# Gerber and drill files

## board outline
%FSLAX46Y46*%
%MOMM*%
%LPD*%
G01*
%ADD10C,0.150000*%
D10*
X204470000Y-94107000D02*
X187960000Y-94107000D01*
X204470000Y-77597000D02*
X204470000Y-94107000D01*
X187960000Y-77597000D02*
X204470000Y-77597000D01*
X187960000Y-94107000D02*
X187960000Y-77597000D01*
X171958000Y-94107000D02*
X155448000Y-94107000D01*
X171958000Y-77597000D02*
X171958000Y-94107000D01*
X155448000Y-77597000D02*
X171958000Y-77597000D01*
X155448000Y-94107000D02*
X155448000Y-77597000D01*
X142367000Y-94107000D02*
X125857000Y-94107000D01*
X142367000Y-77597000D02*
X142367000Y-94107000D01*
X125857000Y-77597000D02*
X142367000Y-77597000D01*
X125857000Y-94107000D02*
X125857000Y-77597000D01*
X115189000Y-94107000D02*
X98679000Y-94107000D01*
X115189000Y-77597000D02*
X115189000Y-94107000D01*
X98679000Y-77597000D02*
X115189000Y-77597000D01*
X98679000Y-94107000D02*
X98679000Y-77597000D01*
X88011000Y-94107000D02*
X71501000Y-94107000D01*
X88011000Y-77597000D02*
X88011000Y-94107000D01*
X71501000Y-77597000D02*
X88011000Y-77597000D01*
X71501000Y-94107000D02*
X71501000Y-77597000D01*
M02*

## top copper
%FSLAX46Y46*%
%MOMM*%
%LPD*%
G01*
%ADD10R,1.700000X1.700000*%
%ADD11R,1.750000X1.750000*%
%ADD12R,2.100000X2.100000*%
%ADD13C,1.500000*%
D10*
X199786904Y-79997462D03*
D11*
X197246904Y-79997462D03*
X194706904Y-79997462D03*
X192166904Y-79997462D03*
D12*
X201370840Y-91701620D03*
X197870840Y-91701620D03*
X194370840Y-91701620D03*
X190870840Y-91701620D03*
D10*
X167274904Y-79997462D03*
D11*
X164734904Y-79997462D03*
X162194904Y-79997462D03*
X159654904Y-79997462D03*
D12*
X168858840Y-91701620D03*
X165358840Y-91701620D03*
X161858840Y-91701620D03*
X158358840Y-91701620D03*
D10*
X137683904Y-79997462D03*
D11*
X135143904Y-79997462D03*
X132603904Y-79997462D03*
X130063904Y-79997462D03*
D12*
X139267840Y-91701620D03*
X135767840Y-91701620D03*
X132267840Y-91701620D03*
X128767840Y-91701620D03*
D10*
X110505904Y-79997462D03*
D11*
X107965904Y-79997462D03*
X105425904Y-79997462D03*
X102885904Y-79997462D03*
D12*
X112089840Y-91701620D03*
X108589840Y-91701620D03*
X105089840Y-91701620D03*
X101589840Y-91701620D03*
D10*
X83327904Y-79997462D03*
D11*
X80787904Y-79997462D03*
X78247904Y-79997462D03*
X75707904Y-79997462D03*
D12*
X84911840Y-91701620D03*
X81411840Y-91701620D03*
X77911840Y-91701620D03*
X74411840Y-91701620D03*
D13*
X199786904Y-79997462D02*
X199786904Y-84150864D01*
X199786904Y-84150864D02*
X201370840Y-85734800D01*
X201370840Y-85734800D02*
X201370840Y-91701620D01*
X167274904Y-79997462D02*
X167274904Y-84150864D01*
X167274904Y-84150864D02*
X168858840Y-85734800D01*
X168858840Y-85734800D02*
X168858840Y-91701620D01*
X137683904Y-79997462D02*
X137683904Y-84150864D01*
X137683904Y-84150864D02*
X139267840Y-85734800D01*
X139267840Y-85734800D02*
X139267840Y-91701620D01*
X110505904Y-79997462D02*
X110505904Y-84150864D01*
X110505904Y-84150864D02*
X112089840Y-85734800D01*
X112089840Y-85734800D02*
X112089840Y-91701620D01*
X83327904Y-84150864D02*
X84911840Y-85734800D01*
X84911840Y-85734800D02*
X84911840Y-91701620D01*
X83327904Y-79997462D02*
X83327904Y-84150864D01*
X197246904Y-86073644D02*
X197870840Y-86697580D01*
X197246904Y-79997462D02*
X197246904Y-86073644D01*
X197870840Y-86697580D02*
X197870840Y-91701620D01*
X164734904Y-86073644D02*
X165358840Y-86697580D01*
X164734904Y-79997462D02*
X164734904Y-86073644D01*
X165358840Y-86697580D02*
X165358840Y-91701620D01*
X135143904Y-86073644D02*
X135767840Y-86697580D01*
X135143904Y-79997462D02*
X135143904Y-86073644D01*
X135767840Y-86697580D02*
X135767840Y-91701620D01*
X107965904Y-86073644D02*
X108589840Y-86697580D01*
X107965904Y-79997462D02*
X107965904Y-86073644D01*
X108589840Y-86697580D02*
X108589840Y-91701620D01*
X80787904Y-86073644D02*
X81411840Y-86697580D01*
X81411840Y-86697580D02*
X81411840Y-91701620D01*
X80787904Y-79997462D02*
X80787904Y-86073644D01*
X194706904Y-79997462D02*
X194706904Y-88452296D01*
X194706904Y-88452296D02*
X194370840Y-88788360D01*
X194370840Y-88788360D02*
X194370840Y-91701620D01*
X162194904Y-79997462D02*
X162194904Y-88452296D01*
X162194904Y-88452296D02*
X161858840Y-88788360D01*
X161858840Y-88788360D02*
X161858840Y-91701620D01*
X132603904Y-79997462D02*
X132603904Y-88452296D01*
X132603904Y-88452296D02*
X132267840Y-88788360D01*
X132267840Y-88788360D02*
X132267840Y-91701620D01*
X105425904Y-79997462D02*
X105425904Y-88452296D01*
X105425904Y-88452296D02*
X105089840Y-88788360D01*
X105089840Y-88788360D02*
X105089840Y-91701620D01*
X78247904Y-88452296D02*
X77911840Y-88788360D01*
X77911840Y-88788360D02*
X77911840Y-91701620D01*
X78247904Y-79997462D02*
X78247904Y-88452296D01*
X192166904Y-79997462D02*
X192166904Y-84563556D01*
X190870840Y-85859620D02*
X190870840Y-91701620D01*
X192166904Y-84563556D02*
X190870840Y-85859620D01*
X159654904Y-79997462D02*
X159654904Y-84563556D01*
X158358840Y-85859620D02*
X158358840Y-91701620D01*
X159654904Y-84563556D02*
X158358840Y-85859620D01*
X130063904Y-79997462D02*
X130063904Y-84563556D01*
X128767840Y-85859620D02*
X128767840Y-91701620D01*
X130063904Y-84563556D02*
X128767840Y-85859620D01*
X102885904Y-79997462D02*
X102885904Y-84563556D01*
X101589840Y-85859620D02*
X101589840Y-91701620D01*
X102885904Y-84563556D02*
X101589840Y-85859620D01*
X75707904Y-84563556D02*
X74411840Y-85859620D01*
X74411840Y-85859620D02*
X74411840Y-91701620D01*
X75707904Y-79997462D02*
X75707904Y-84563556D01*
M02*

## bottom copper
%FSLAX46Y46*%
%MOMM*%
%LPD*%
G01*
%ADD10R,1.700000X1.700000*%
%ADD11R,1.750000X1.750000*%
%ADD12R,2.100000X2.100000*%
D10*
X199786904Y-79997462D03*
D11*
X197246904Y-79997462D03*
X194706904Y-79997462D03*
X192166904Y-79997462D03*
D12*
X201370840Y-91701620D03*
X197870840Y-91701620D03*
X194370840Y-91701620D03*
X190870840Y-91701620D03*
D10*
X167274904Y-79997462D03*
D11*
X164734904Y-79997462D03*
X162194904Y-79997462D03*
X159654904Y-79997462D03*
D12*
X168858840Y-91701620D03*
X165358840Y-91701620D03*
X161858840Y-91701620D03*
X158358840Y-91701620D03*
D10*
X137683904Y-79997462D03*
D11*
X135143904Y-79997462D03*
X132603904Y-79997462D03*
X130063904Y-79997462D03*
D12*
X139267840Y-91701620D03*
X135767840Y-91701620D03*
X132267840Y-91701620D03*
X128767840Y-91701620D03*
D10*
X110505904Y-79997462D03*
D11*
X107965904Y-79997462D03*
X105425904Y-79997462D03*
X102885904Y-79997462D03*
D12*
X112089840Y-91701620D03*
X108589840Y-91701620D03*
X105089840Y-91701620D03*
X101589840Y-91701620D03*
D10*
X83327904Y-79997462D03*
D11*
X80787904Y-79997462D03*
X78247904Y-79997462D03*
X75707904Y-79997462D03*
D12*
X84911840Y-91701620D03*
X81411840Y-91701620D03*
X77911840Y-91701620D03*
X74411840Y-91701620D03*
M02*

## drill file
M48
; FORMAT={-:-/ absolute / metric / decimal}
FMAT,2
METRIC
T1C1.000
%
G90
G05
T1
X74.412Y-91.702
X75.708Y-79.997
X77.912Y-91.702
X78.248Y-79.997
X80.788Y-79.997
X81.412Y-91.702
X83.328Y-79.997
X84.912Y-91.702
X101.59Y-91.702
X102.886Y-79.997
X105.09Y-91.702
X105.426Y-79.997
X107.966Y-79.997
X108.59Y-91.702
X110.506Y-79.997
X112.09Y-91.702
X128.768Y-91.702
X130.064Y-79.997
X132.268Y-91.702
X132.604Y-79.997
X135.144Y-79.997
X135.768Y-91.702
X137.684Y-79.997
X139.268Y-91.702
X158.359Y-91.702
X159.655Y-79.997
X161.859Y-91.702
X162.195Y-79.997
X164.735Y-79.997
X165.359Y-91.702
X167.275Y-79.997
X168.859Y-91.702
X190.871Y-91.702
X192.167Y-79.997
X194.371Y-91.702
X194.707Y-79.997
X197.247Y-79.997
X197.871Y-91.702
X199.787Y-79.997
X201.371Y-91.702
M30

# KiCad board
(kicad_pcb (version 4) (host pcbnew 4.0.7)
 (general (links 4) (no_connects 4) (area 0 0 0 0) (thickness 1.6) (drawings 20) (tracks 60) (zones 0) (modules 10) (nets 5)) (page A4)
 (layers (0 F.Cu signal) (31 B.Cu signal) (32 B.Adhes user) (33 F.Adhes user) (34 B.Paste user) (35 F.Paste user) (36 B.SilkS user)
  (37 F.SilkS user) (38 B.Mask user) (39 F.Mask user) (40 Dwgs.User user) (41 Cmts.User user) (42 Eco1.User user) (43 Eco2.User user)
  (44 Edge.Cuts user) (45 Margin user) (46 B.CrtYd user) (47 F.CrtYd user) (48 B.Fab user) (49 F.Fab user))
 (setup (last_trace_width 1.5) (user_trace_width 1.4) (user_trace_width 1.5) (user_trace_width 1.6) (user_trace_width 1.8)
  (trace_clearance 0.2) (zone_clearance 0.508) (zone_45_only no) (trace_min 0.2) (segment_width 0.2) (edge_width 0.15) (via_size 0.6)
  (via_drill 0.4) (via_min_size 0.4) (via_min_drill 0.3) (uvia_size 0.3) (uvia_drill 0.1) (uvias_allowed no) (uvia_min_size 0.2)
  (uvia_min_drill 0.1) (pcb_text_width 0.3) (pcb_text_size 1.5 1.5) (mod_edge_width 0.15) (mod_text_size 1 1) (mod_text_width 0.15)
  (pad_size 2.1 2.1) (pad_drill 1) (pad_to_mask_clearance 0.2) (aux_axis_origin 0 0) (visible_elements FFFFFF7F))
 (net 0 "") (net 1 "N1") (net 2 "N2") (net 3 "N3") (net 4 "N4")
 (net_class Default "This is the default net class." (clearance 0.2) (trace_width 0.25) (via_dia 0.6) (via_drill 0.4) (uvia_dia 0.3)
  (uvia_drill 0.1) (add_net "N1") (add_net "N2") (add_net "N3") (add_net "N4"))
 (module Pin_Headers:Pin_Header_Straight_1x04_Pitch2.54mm (layer F.Cu) (at 199.786904 79.997462 270)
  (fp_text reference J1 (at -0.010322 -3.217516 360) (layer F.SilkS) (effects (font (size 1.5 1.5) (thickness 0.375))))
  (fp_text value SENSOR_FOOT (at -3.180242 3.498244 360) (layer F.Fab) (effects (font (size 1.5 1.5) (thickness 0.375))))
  (pad 1 thru_hole rect (at 0 0 270) (size 1.7 1.7) (drill 1) (layers *.Cu *.Mask) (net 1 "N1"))
  (pad 2 thru_hole rect (at 0 2.54 270) (size 1.75 1.75) (drill 1) (layers *.Cu *.Mask) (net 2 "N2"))
  (pad 3 thru_hole rect (at 0 5.08 270) (size 1.75 1.75) (drill 1) (layers *.Cu *.Mask) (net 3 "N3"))
  (pad 4 thru_hole rect (at 0 7.62 270) (size 1.75 1.75) (drill 1) (layers *.Cu *.Mask) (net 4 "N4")))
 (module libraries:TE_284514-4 (layer F.Cu) (at 196.12084 91.70162 180)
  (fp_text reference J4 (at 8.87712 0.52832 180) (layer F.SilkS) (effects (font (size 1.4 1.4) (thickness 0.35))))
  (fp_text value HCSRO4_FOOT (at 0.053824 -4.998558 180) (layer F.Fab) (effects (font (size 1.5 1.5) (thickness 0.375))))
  (pad 1 thru_hole rect (at -5.25 0 180) (size 2.1 2.1) (drill 1) (layers *.Cu *.Mask) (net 1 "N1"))
  (pad 2 thru_hole rect (at -1.75 0 180) (size 2.1 2.1) (drill 1) (layers *.Cu *.Mask) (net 2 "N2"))
  (pad 3 thru_hole rect (at 1.75 0 180) (size 2.1 2.1) (drill 1) (layers *.Cu *.Mask) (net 3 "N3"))
  (pad 4 thru_hole rect (at 5.25 0 180) (size 2.1 2.1) (drill 1) (layers *.Cu *.Mask) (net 4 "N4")))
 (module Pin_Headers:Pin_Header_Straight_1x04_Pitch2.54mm (layer F.Cu) (at 167.274904 79.997462 270)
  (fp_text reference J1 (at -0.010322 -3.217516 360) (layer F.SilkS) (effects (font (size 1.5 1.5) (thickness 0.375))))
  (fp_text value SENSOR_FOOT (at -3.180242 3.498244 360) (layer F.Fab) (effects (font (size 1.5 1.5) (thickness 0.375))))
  (pad 1 thru_hole rect (at 0 0 270) (size 1.7 1.7) (drill 1) (layers *.Cu *.Mask) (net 1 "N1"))
  (pad 2 thru_hole rect (at 0 2.54 270) (size 1.75 1.75) (drill 1) (layers *.Cu *.Mask) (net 2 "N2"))
  (pad 3 thru_hole rect (at 0 5.08 270) (size 1.75 1.75) (drill 1) (layers *.Cu *.Mask) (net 3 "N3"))
  (pad 4 thru_hole rect (at 0 7.62 270) (size 1.75 1.75) (drill 1) (layers *.Cu *.Mask) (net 4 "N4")))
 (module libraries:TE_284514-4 (layer F.Cu) (at 163.60884 91.70162 180)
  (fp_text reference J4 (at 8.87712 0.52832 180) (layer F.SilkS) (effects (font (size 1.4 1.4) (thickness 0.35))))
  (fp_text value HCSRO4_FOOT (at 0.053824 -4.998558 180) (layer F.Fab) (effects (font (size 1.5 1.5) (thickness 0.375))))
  (pad 1 thru_hole rect (at -5.25 0 180) (size 2.1 2.1) (drill 1) (layers *.Cu *.Mask) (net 1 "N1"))
  (pad 2 thru_hole rect (at -1.75 0 180) (size 2.1 2.1) (drill 1) (layers *.Cu *.Mask) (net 2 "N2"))
  (pad 3 thru_hole rect (at 1.75 0 180) (size 2.1 2.1) (drill 1) (layers *.Cu *.Mask) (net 3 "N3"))
  (pad 4 thru_hole rect (at 5.25 0 180) (size 2.1 2.1) (drill 1) (layers *.Cu *.Mask) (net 4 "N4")))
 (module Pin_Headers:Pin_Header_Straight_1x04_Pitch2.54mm (layer F.Cu) (at 137.683904 79.997462 270)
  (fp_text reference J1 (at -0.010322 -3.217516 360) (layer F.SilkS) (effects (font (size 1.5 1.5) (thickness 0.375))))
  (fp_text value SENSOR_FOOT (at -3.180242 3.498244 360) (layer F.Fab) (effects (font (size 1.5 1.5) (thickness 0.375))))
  (pad 1 thru_hole rect (at 0 0 270) (size 1.7 1.7) (drill 1) (layers *.Cu *.Mask) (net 1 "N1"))
  (pad 2 thru_hole rect (at 0 2.54 270) (size 1.75 1.75) (drill 1) (layers *.Cu *.Mask) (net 2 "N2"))
  (pad 3 thru_hole rect (at 0 5.08 270) (size 1.75 1.75) (drill 1) (layers *.Cu *.Mask) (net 3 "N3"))
  (pad 4 thru_hole rect (at 0 7.62 270) (size 1.75 1.75) (drill 1) (layers *.Cu *.Mask) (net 4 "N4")))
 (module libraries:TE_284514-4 (layer F.Cu) (at 134.01784 91.70162 180)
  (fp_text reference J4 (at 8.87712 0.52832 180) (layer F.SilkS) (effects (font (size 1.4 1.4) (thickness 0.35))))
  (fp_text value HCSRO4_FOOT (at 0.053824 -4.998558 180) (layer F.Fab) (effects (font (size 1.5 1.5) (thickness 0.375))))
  (pad 1 thru_hole rect (at -5.25 0 180) (size 2.1 2.1) (drill 1) (layers *.Cu *.Mask) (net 1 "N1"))
  (pad 2 thru_hole rect (at -1.75 0 180) (size 2.1 2.1) (drill 1) (layers *.Cu *.Mask) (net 2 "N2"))
  (pad 3 thru_hole rect (at 1.75 0 180) (size 2.1 2.1) (drill 1) (layers *.Cu *.Mask) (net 3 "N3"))
  (pad 4 thru_hole rect (at 5.25 0 180) (size 2.1 2.1) (drill 1) (layers *.Cu *.Mask) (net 4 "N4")))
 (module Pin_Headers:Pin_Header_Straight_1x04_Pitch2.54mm (layer F.Cu) (at 110.505904 79.997462 270)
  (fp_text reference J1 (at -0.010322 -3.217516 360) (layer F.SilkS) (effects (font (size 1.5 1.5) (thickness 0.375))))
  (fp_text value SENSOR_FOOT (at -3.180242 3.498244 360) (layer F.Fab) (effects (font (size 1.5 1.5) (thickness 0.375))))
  (pad 1 thru_hole rect (at 0 0 270) (size 1.7 1.7) (drill 1) (layers *.Cu *.Mask) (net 1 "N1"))
  (pad 2 thru_hole rect (at 0 2.54 270) (size 1.75 1.75) (drill 1) (layers *.Cu *.Mask) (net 2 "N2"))
  (pad 3 thru_hole rect (at 0 5.08 270) (size 1.75 1.75) (drill 1) (layers *.Cu *.Mask) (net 3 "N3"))
  (pad 4 thru_hole rect (at 0 7.62 270) (size 1.75 1.75) (drill 1) (layers *.Cu *.Mask) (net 4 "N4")))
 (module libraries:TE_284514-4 (layer F.Cu) (at 106.83984 91.70162 180)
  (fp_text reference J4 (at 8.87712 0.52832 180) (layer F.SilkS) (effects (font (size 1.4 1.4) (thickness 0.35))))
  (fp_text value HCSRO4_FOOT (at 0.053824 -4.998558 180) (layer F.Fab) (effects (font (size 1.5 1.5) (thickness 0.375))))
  (pad 1 thru_hole rect (at -5.25 0 180) (size 2.1 2.1) (drill 1) (layers *.Cu *.Mask) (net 1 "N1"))
  (pad 2 thru_hole rect (at -1.75 0 180) (size 2.1 2.1) (drill 1) (layers *.Cu *.Mask) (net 2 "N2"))
  (pad 3 thru_hole rect (at 1.75 0 180) (size 2.1 2.1) (drill 1) (layers *.Cu *.Mask) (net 3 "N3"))
  (pad 4 thru_hole rect (at 5.25 0 180) (size 2.1 2.1) (drill 1) (layers *.Cu *.Mask) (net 4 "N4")))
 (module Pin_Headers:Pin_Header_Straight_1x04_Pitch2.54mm (layer F.Cu) (at 83.327904 79.997462 270)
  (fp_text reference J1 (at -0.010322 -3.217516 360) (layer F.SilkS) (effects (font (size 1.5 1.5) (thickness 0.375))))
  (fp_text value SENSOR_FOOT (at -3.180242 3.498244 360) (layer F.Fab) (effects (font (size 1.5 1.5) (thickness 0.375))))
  (pad 1 thru_hole rect (at 0 0 270) (size 1.7 1.7) (drill 1) (layers *.Cu *.Mask) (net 1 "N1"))
  (pad 2 thru_hole rect (at 0 2.54 270) (size 1.75 1.75) (drill 1) (layers *.Cu *.Mask) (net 2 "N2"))
  (pad 3 thru_hole rect (at 0 5.08 270) (size 1.75 1.75) (drill 1) (layers *.Cu *.Mask) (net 3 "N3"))
  (pad 4 thru_hole rect (at 0 7.62 270) (size 1.75 1.75) (drill 1) (layers *.Cu *.Mask) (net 4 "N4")))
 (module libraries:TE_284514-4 (layer F.Cu) (at 79.66184 91.70162 180)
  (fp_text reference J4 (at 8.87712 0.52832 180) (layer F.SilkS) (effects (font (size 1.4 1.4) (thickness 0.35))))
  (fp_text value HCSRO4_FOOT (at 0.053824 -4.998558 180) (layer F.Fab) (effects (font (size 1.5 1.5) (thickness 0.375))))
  (pad 1 thru_hole rect (at -5.25 0 180) (size 2.1 2.1) (drill 1) (layers *.Cu *.Mask) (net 1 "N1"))
  (pad 2 thru_hole rect (at -1.75 0 180) (size 2.1 2.1) (drill 1) (layers *.Cu *.Mask) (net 2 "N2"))
  (pad 3 thru_hole rect (at 1.75 0 180) (size 2.1 2.1) (drill 1) (layers *.Cu *.Mask) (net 3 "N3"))
  (pad 4 thru_hole rect (at 5.25 0 180) (size 2.1 2.1) (drill 1) (layers *.Cu *.Mask) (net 4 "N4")))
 (gr_line (start 204.47 94.107) (end 187.96 94.107) (layer Edge.Cuts) (width 0.15))
 (gr_line (start 204.47 77.597) (end 204.47 94.107) (layer Edge.Cuts) (width 0.15))
 (gr_line (start 187.96 77.597) (end 204.47 77.597) (layer Edge.Cuts) (width 0.15))
 (gr_line (start 187.96 94.107) (end 187.96 77.597) (layer Edge.Cuts) (width 0.15))
 (gr_line (start 171.958 94.107) (end 155.448 94.107) (layer Edge.Cuts) (width 0.15))
 (gr_line (start 171.958 77.597) (end 171.958 94.107) (layer Edge.Cuts) (width 0.15))
 (gr_line (start 155.448 77.597) (end 171.958 77.597) (layer Edge.Cuts) (width 0.15))
 (gr_line (start 155.448 94.107) (end 155.448 77.597) (layer Edge.Cuts) (width 0.15))
 (gr_line (start 142.367 94.107) (end 125.857 94.107) (layer Edge.Cuts) (width 0.15))
 (gr_line (start 142.367 77.597) (end 142.367 94.107) (layer Edge.Cuts) (width 0.15))
 (gr_line (start 125.857 77.597) (end 142.367 77.597) (layer Edge.Cuts) (width 0.15))
 (gr_line (start 125.857 94.107) (end 125.857 77.597) (layer Edge.Cuts) (width 0.15))
 (gr_line (start 115.189 94.107) (end 98.679 94.107) (layer Edge.Cuts) (width 0.15))
 (gr_line (start 115.189 77.597) (end 115.189 94.107) (layer Edge.Cuts) (width 0.15))
 (gr_line (start 98.679 77.597) (end 115.189 77.597) (layer Edge.Cuts) (width 0.15))
 (gr_line (start 98.679 94.107) (end 98.679 77.597) (layer Edge.Cuts) (width 0.15))
 (gr_line (start 88.011 94.107) (end 71.501 94.107) (layer Edge.Cuts) (width 0.15))
 (gr_line (start 88.011 77.597) (end 88.011 94.107) (layer Edge.Cuts) (width 0.15))
 (gr_line (start 71.501 77.597) (end 88.011 77.597) (layer Edge.Cuts) (width 0.15))
 (gr_line (start 71.501 94.107) (end 71.501 77.597) (layer Edge.Cuts) (width 0.15))
 (segment (start 199.786904 79.997462) (end 199.786904 84.150864) (width 1.5) (layer F.Cu) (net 1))
 (segment (start 199.786904 84.150864) (end 201.37084 85.7348) (width 1.5) (layer F.Cu) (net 1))
 (segment (start 201.37084 85.7348) (end 201.37084 91.70162) (width 1.5) (layer F.Cu) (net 1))
 (segment (start 167.274904 79.997462) (end 167.274904 84.150864) (width 1.5) (layer F.Cu) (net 1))
 (segment (start 167.274904 84.150864) (end 168.85884 85.7348) (width 1.5) (layer F.Cu) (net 1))
 (segment (start 168.85884 85.7348) (end 168.85884 91.70162) (width 1.5) (layer F.Cu) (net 1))
 (segment (start 137.683904 79.997462) (end 137.683904 84.150864) (width 1.5) (layer F.Cu) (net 1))
 (segment (start 137.683904 84.150864) (end 139.26784 85.7348) (width 1.5) (layer F.Cu) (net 1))
 (segment (start 139.26784 85.7348) (end 139.26784 91.70162) (width 1.5) (layer F.Cu) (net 1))
 (segment (start 110.505904 79.997462) (end 110.505904 84.150864) (width 1.5) (layer F.Cu) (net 1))
 (segment (start 110.505904 84.150864) (end 112.08984 85.7348) (width 1.5) (layer F.Cu) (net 1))
 (segment (start 112.08984 85.7348) (end 112.08984 91.70162) (width 1.5) (layer F.Cu) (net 1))
 (segment (start 83.327904 84.150864) (end 84.91184 85.7348) (width 1.5) (layer F.Cu) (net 1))
 (segment (start 84.91184 85.7348) (end 84.91184 91.70162) (width 1.5) (layer F.Cu) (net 1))
 (segment (start 83.327904 79.997462) (end 83.327904 84.150864) (width 1.5) (layer F.Cu) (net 1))
 (segment (start 197.246904 86.073644) (end 197.87084 86.69758) (width 1.5) (layer F.Cu) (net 2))
 (segment (start 197.246904 79.997462) (end 197.246904 86.073644) (width 1.5) (layer F.Cu) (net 2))
 (segment (start 197.87084 86.69758) (end 197.87084 91.70162) (width 1.5) (layer F.Cu) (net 2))
 (segment (start 164.734904 86.073644) (end 165.35884 86.69758) (width 1.5) (layer F.Cu) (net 2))
 (segment (start 164.734904 79.997462) (end 164.734904 86.073644) (width 1.5) (layer F.Cu) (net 2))
 (segment (start 165.35884 86.69758) (end 165.35884 91.70162) (width 1.5) (layer F.Cu) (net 2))
 (segment (start 135.143904 86.073644) (end 135.76784 86.69758) (width 1.5) (layer F.Cu) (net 2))
 (segment (start 135.143904 79.997462) (end 135.143904 86.073644) (width 1.5) (layer F.Cu) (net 2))
 (segment (start 135.76784 86.69758) (end 135.76784 91.70162) (width 1.5) (layer F.Cu) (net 2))
 (segment (start 107.965904 86.073644) (end 108.58984 86.69758) (width 1.5) (layer F.Cu) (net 2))
 (segment (start 107.965904 79.997462) (end 107.965904 86.073644) (width 1.5) (layer F.Cu) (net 2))
 (segment (start 108.58984 86.69758) (end 108.58984 91.70162) (width 1.5) (layer F.Cu) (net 2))
 (segment (start 80.787904 86.073644) (end 81.41184 86.69758) (width 1.5) (layer F.Cu) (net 2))
 (segment (start 81.41184 86.69758) (end 81.41184 91.70162) (width 1.5) (layer F.Cu) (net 2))
 (segment (start 80.787904 79.997462) (end 80.787904 86.073644) (width 1.5) (layer F.Cu) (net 2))
 (segment (start 194.706904 79.997462) (end 194.706904 88.452296) (width 1.5) (layer F.Cu) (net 3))
 (segment (start 194.706904 88.452296) (end 194.37084 88.78836) (width 1.5) (layer F.Cu) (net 3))
 (segment (start 194.37084 88.78836) (end 194.37084 91.70162) (width 1.5) (layer F.Cu) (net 3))
 (segment (start 162.194904 79.997462) (end 162.194904 88.452296) (width 1.5) (layer F.Cu) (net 3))
 (segment (start 162.194904 88.452296) (end 161.85884 88.78836) (width 1.5) (layer F.Cu) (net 3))
 (segment (start 161.85884 88.78836) (end 161.85884 91.70162) (width 1.5) (layer F.Cu) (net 3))
 (segment (start 132.603904 79.997462) (end 132.603904 88.452296) (width 1.5) (layer F.Cu) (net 3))
 (segment (start 132.603904 88.452296) (end 132.26784 88.78836) (width 1.5) (layer F.Cu) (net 3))
 (segment (start 132.26784 88.78836) (end 132.26784 91.70162) (width 1.5) (layer F.Cu) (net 3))
 (segment (start 105.425904 79.997462) (end 105.425904 88.452296) (width 1.5) (layer F.Cu) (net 3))
 (segment (start 105.425904 88.452296) (end 105.08984 88.78836) (width 1.5) (layer F.Cu) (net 3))
 (segment (start 105.08984 88.78836) (end 105.08984 91.70162) (width 1.5) (layer F.Cu) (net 3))
 (segment (start 78.247904 88.452296) (end 77.91184 88.78836) (width 1.5) (layer F.Cu) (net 3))
 (segment (start 77.91184 88.78836) (end 77.91184 91.70162) (width 1.5) (layer F.Cu) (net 3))
 (segment (start 78.247904 79.997462) (end 78.247904 88.452296) (width 1.5) (layer F.Cu) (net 3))
 (segment (start 192.166904 79.997462) (end 192.166904 84.563556) (width 1.5) (layer F.Cu) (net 4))
 (segment (start 190.87084 85.85962) (end 190.87084 91.70162) (width 1.5) (layer F.Cu) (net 4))
 (segment (start 192.166904 84.563556) (end 190.87084 85.85962) (width 1.5) (layer F.Cu) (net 4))
 (segment (start 159.654904 79.997462) (end 159.654904 84.563556) (width 1.5) (layer F.Cu) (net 4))
 (segment (start 158.35884 85.85962) (end 158.35884 91.70162) (width 1.5) (layer F.Cu) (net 4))
 (segment (start 159.654904 84.563556) (end 158.35884 85.85962) (width 1.5) (layer F.Cu) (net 4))
 (segment (start 130.063904 79.997462) (end 130.063904 84.563556) (width 1.5) (layer F.Cu) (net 4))
 (segment (start 128.76784 85.85962) (end 128.76784 91.70162) (width 1.5) (layer F.Cu) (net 4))
 (segment (start 130.063904 84.563556) (end 128.76784 85.85962) (width 1.5) (layer F.Cu) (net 4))
 (segment (start 102.885904 79.997462) (end 102.885904 84.563556) (width 1.5) (layer F.Cu) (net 4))
 (segment (start 101.58984 85.85962) (end 101.58984 91.70162) (width 1.5) (layer F.Cu) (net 4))
 (segment (start 102.885904 84.563556) (end 101.58984 85.85962) (width 1.5) (layer F.Cu) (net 4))
 (segment (start 75.707904 84.563556) (end 74.41184 85.85962) (width 1.5) (layer F.Cu) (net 4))
 (segment (start 74.41184 85.85962) (end 74.41184 91.70162) (width 1.5) (layer F.Cu) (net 4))
 (segment (start 75.707904 79.997462) (end 75.707904 84.563556) (width 1.5) (layer F.Cu) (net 4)))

